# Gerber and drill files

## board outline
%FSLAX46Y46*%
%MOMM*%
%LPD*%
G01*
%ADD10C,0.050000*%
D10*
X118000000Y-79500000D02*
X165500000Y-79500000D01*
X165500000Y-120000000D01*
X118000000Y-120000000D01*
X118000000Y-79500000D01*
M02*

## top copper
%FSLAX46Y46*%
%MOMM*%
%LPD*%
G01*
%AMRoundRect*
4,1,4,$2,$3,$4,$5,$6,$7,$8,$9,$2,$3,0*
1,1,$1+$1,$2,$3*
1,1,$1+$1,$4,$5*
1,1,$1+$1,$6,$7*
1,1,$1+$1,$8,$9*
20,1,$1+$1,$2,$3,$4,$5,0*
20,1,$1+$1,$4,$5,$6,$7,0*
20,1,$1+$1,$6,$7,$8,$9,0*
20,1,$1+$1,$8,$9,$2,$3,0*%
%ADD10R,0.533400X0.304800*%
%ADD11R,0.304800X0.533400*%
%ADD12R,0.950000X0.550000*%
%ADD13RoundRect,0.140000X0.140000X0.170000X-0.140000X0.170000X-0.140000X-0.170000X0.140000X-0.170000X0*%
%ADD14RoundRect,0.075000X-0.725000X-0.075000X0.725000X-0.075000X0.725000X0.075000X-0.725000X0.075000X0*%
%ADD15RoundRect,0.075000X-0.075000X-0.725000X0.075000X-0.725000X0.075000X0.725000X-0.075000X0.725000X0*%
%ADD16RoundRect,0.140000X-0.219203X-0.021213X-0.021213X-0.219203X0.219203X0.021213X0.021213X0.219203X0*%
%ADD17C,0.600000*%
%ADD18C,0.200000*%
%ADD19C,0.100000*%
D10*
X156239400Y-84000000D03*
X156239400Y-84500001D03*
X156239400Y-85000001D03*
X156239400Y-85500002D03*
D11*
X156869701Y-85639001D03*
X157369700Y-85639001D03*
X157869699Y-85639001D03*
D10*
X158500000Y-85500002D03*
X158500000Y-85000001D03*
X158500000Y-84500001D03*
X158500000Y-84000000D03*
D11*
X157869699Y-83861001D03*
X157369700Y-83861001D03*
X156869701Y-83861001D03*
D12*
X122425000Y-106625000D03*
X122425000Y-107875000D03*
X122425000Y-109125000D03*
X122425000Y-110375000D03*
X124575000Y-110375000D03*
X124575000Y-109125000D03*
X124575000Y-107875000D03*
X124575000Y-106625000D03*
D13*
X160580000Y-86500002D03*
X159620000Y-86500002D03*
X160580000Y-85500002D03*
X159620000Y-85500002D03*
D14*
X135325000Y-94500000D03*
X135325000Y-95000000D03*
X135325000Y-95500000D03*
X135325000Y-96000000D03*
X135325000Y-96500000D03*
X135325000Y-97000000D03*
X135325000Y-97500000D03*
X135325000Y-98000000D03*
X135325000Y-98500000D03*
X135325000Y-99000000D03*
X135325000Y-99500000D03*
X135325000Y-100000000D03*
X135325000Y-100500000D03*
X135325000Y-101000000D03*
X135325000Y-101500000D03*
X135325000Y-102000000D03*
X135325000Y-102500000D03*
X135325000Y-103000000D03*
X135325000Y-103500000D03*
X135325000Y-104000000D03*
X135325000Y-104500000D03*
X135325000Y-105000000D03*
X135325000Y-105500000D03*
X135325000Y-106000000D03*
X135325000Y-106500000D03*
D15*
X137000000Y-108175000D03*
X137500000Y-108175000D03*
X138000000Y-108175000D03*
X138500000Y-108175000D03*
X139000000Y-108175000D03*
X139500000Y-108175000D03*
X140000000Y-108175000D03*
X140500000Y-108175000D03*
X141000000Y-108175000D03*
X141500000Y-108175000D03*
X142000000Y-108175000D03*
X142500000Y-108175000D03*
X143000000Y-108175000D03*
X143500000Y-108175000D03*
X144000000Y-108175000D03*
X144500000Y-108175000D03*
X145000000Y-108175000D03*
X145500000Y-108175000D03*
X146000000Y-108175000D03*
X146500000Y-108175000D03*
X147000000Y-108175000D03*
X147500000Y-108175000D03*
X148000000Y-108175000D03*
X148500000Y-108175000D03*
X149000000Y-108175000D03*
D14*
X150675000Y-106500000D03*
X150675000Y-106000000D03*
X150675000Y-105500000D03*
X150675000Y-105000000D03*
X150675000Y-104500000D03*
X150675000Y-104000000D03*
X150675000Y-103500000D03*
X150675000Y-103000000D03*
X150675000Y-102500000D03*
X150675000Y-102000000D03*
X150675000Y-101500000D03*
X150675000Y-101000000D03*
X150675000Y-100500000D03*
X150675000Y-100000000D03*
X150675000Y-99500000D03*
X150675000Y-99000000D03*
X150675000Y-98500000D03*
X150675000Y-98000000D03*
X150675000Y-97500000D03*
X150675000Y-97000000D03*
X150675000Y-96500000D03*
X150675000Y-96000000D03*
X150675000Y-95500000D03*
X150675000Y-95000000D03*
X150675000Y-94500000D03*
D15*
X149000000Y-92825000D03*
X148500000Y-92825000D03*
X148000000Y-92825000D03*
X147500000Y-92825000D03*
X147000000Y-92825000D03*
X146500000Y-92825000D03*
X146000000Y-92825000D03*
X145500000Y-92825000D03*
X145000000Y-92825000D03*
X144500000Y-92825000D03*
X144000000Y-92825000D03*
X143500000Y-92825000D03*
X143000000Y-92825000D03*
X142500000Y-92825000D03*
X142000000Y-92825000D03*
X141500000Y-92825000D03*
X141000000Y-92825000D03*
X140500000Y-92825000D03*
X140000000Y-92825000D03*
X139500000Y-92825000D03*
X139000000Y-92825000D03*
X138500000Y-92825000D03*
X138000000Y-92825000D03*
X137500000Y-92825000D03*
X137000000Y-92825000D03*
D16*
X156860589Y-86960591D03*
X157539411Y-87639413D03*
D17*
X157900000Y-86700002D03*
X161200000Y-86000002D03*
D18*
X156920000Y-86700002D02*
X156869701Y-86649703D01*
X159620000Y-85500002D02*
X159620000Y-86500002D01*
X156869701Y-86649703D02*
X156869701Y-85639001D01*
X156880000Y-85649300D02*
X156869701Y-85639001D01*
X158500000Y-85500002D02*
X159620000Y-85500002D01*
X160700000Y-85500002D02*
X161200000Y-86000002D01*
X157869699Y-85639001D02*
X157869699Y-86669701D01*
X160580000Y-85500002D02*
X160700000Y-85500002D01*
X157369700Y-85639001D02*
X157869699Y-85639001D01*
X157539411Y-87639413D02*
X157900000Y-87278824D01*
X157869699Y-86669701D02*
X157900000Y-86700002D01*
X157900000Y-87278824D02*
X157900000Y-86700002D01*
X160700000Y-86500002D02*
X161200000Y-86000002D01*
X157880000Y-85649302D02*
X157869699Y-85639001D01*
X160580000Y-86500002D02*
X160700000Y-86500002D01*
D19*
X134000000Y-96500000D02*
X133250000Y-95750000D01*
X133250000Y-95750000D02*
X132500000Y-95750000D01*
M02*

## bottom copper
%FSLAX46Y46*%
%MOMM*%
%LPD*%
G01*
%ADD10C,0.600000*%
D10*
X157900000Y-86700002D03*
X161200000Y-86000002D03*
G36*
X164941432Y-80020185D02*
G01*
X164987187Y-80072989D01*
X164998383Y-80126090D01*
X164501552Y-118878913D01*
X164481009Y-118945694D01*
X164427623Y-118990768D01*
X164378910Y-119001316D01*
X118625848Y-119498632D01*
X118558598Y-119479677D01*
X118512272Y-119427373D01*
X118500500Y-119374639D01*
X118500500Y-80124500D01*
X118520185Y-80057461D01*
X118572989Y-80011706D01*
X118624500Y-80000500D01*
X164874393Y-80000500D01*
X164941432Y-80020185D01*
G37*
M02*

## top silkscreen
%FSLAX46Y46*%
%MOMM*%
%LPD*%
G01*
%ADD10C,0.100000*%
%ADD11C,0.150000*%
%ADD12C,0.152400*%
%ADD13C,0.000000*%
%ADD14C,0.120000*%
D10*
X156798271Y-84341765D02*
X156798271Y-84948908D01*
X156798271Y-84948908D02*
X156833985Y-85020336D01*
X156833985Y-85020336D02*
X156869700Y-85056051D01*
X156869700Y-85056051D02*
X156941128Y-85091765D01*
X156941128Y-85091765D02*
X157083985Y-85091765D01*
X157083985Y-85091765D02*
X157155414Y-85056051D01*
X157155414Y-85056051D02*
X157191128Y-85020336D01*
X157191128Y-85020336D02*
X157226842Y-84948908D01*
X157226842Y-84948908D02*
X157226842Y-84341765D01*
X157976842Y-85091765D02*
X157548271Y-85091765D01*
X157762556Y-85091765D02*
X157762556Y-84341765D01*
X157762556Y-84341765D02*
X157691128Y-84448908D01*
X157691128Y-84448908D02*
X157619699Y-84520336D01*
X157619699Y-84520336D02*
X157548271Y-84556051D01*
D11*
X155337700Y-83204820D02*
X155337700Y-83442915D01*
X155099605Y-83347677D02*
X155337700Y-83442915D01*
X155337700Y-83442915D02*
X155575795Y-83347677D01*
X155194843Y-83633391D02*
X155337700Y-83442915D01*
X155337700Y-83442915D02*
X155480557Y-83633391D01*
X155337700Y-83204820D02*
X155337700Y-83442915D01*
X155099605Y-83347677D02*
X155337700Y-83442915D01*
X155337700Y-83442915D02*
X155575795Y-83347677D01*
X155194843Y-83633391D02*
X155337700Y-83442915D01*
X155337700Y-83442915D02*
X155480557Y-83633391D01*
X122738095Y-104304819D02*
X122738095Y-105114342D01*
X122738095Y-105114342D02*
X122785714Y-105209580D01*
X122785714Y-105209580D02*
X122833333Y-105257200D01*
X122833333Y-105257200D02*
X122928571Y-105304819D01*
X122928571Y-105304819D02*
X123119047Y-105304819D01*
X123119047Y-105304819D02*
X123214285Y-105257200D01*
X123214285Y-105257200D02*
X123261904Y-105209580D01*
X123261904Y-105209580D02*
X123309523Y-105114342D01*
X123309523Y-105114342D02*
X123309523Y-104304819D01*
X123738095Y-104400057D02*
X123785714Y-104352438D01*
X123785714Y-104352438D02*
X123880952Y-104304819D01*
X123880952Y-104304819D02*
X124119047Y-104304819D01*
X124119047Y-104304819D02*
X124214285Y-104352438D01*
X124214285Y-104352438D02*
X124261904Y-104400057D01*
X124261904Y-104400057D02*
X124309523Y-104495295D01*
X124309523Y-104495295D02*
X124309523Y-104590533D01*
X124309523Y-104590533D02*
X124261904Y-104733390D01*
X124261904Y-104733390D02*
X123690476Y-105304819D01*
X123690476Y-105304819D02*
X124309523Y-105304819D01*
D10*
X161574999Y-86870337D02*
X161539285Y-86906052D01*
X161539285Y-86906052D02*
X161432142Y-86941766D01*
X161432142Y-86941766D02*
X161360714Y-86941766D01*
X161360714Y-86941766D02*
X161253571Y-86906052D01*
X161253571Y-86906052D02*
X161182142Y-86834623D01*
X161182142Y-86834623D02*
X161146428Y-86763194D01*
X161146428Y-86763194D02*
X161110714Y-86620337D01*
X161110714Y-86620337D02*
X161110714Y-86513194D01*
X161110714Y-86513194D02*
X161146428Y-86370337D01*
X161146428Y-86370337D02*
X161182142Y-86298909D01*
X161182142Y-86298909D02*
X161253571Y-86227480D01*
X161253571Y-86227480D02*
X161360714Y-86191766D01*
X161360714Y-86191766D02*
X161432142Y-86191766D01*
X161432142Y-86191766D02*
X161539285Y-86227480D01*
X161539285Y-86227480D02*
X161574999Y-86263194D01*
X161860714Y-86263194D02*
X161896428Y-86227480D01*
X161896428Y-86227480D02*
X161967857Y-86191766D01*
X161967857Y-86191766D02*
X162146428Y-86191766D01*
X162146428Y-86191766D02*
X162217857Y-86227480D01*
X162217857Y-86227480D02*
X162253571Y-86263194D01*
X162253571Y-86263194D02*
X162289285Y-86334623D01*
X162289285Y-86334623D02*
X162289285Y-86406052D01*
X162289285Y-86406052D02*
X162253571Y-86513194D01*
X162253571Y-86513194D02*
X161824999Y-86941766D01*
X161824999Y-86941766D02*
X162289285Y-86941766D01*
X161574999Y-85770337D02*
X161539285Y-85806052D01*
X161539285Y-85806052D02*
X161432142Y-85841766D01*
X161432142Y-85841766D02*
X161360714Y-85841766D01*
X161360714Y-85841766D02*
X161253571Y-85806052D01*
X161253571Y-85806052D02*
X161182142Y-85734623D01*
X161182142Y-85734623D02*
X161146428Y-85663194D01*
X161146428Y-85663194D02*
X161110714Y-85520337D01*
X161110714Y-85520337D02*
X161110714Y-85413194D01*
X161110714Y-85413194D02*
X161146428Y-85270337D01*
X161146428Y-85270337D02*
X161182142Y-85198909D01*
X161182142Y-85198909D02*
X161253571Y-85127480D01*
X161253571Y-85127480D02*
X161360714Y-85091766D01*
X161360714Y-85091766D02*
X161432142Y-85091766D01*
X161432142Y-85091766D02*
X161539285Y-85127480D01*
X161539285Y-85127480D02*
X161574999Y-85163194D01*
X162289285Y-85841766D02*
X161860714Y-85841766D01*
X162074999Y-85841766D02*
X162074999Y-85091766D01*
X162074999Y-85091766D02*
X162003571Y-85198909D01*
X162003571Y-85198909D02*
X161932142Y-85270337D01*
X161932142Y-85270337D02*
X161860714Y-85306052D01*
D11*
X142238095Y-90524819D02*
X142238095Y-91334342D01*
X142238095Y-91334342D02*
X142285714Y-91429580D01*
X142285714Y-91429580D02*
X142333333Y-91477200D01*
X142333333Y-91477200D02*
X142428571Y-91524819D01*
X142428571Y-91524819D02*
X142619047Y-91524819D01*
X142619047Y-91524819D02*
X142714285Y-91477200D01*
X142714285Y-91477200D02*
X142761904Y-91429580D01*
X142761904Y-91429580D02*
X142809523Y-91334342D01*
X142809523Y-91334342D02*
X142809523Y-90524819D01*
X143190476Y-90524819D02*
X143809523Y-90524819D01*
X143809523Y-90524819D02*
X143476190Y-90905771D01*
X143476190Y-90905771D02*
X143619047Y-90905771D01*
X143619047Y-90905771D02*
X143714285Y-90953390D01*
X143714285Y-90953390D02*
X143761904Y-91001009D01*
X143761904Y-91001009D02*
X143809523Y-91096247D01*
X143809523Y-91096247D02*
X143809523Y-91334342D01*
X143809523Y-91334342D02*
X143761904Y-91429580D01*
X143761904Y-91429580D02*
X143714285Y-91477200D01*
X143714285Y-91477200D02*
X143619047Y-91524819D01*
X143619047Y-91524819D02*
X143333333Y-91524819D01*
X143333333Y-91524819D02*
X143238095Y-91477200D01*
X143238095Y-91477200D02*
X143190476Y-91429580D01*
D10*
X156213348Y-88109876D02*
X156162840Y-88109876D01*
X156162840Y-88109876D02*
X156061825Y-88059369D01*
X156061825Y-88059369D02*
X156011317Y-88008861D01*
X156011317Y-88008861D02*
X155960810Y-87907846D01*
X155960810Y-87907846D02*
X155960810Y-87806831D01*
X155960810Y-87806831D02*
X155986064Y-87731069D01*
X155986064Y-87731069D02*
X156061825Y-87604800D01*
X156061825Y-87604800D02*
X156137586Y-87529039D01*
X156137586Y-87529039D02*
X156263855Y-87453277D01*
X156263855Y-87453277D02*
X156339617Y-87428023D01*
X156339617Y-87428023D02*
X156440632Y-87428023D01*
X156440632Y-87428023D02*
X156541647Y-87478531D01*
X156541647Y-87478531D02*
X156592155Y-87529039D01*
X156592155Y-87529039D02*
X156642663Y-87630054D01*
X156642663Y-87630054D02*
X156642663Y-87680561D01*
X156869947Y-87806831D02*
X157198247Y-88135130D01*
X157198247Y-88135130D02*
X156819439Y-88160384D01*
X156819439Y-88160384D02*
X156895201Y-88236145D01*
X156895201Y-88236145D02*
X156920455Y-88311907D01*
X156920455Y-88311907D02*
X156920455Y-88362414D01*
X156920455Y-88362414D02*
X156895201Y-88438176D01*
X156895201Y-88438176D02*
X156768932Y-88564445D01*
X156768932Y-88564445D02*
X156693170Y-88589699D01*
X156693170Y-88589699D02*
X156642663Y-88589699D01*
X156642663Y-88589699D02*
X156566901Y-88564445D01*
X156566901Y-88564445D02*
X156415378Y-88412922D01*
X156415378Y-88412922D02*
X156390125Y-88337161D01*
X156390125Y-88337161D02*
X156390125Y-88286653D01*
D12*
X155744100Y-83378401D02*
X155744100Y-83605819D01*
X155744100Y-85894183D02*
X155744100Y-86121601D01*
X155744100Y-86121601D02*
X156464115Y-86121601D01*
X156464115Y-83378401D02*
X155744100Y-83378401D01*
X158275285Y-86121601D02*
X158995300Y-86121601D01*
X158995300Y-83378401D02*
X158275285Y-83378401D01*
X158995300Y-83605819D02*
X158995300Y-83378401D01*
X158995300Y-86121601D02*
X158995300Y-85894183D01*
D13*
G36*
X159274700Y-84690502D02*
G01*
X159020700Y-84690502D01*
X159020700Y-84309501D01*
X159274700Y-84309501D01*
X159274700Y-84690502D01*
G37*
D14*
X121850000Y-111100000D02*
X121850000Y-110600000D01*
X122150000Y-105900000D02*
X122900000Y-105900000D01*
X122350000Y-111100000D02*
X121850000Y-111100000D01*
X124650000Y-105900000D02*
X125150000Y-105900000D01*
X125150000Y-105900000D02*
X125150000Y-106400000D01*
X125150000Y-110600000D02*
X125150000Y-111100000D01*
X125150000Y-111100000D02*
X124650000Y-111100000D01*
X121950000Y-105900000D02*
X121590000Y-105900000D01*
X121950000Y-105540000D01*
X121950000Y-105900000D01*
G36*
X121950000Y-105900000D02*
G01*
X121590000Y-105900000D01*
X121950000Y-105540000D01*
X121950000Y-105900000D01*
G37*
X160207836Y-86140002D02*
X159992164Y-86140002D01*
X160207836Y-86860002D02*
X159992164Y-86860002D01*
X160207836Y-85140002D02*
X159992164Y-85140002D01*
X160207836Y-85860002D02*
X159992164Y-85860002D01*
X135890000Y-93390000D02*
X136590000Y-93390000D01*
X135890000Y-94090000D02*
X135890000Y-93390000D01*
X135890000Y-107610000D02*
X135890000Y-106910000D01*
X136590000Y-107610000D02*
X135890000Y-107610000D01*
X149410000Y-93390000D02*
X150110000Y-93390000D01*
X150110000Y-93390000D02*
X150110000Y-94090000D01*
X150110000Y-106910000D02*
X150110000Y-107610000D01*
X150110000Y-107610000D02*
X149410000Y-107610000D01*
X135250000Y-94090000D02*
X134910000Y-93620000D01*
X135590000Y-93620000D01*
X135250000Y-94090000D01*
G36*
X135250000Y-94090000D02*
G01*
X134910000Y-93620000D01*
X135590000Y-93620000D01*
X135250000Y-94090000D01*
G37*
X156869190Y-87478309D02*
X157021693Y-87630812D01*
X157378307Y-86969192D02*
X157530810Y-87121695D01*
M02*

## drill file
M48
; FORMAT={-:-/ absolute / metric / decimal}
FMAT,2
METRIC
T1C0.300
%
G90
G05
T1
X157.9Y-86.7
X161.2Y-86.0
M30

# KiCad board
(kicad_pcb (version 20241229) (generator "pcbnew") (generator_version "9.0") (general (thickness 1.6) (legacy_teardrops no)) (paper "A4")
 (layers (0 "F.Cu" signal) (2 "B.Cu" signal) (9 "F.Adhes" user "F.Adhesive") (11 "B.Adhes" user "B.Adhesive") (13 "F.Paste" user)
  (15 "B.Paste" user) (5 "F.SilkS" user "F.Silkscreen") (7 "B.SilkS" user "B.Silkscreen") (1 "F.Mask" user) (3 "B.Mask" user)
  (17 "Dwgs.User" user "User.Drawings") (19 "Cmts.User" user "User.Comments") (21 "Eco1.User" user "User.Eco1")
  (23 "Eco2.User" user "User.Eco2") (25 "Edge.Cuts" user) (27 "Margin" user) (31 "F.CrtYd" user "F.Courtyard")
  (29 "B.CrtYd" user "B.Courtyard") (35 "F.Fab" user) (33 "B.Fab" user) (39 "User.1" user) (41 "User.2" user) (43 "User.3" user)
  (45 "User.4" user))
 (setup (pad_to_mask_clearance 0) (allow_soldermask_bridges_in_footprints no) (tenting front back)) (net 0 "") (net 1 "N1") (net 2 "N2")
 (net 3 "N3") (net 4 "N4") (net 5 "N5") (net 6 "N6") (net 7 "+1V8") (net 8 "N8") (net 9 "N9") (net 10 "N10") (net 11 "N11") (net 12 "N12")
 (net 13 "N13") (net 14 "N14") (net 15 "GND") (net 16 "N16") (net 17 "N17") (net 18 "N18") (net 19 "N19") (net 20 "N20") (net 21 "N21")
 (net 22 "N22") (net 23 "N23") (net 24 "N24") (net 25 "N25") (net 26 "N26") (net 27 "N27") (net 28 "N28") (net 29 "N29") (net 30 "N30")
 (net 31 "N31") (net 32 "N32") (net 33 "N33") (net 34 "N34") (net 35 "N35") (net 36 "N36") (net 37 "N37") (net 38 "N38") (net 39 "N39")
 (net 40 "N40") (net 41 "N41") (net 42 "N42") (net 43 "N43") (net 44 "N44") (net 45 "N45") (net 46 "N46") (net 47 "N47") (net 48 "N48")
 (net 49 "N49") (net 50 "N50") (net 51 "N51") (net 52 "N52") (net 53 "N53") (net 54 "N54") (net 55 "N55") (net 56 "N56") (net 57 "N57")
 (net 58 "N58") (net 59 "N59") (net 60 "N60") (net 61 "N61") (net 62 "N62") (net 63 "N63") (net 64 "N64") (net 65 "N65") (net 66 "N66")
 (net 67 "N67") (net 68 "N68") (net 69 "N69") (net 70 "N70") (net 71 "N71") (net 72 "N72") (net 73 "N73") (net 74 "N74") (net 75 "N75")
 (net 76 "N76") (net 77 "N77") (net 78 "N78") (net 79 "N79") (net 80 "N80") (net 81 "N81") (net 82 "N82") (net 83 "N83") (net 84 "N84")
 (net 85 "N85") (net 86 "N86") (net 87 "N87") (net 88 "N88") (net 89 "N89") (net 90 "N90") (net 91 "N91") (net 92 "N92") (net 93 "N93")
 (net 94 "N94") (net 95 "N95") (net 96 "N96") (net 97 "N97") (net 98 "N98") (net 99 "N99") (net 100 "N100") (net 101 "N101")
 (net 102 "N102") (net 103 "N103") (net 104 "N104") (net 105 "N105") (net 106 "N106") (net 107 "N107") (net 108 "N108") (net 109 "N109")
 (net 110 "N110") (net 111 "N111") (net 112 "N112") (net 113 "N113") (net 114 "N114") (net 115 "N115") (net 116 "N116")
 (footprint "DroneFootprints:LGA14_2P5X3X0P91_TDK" (layer "F.Cu") (at 157.3697 84.750001)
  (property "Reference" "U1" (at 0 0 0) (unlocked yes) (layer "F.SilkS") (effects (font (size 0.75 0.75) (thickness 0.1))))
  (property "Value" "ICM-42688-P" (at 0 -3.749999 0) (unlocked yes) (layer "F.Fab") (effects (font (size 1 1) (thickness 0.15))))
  (fp_line (start -1.6256 -1.3716) (end -1.6256 -1.144182) (stroke (width 0.1524) (type solid)) (layer "F.SilkS"))
  (fp_line (start -1.6256 1.144182) (end -1.6256 1.3716) (stroke (width 0.1524) (type solid)) (layer "F.SilkS"))
  (fp_line (start -1.6256 1.3716) (end -0.905585 1.3716) (stroke (width 0.1524) (type solid)) (layer "F.SilkS"))
  (fp_line (start -0.905585 -1.3716) (end -1.6256 -1.3716) (stroke (width 0.1524) (type solid)) (layer "F.SilkS"))
  (fp_line (start 0.905585 1.3716) (end 1.6256 1.3716) (stroke (width 0.1524) (type solid)) (layer "F.SilkS"))
  (fp_line (start 1.6256 -1.3716) (end 0.905585 -1.3716) (stroke (width 0.1524) (type solid)) (layer "F.SilkS"))
  (fp_line (start 1.6256 -1.144182) (end 1.6256 -1.3716) (stroke (width 0.1524) (type solid)) (layer "F.SilkS"))
  (fp_line (start 1.6256 1.3716) (end 1.6256 1.144182) (stroke (width 0.1524) (type solid)) (layer "F.SilkS"))
  (fp_poly
   (pts (xy 1.905 -0.4405) (xy 1.905 -0.059499) (xy 1.651 -0.059499) (xy 1.651 -0.4405)) (stroke (width 0) (type solid)) (fill yes)
   (layer "F.SilkS"))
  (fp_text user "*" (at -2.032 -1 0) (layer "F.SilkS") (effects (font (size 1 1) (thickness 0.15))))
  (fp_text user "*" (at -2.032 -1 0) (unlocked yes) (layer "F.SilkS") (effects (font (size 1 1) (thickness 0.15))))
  (pad "1" smd rect (at -1.1303 -0.750001 90) (size 0.3048 0.5334) (layers "F.Cu" "F.Mask" "F.Paste") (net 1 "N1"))
  (pad "2" smd rect (at -1.1303 -0.25 90) (size 0.3048 0.5334) (layers "F.Cu" "F.Mask" "F.Paste") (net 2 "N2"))
  (pad "3" smd rect (at -1.1303 0.25 90) (size 0.3048 0.5334) (layers "F.Cu" "F.Mask" "F.Paste") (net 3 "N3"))
  (pad "4" smd rect (at -1.1303 0.750001 90) (size 0.3048 0.5334) (layers "F.Cu" "F.Mask" "F.Paste") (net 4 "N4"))
  (pad "5" smd rect (at -0.499999 0.889) (size 0.3048 0.5334) (layers "F.Cu" "F.Mask" "F.Paste") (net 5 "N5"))
  (pad "6" smd rect (at 0 0.889) (size 0.3048 0.5334) (layers "F.Cu" "F.Mask" "F.Paste") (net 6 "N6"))
  (pad "7" smd rect (at 0.499999 0.889) (size 0.3048 0.5334) (layers "F.Cu" "F.Mask" "F.Paste") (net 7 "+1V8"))
  (pad "8" smd rect (at 1.1303 0.750001 90) (size 0.3048 0.5334) (layers "F.Cu" "F.Mask" "F.Paste") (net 7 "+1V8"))
  (pad "9" smd rect (at 1.1303 0.25 90) (size 0.3048 0.5334) (layers "F.Cu" "F.Mask" "F.Paste") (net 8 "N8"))
  (pad "10" smd rect (at 1.1303 -0.25 90) (size 0.3048 0.5334) (layers "F.Cu" "F.Mask" "F.Paste") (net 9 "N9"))
  (pad "11" smd rect (at 1.1303 -0.750001 90) (size 0.3048 0.5334) (layers "F.Cu" "F.Mask" "F.Paste") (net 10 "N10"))
  (pad "12" smd rect (at 0.499999 -0.889) (size 0.3048 0.5334) (layers "F.Cu" "F.Mask" "F.Paste") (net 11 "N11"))
  (pad "13" smd rect (at 0 -0.889) (size 0.3048 0.5334) (layers "F.Cu" "F.Mask" "F.Paste") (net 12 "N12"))
  (pad "14" smd rect (at -0.499999 -0.889) (size 0.3048 0.5334) (layers "F.Cu" "F.Mask" "F.Paste") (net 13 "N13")))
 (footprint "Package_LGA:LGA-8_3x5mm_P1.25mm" (layer "F.Cu") (at 123.5 108.5)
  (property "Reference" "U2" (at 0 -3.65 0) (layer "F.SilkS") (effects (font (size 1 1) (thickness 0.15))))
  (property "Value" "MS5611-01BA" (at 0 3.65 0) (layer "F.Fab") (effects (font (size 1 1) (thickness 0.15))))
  (fp_line (start -1.65 2.6) (end -1.65 2.1) (stroke (width 0.12) (type solid)) (layer "F.SilkS"))
  (fp_line (start -1.35 -2.6) (end -0.6 -2.6) (stroke (width 0.12) (type solid)) (layer "F.SilkS"))
  (fp_line (start -1.15 2.6) (end -1.65 2.6) (stroke (width 0.12) (type solid)) (layer "F.SilkS"))
  (fp_line (start 1.15 -2.6) (end 1.65 -2.6) (stroke (width 0.12) (type solid)) (layer "F.SilkS"))
  (fp_line (start 1.65 -2.6) (end 1.65 -2.1) (stroke (width 0.12) (type solid)) (layer "F.SilkS"))
  (fp_line (start 1.65 2.1) (end 1.65 2.6) (stroke (width 0.12) (type solid)) (layer "F.SilkS"))
  (fp_line (start 1.65 2.6) (end 1.15 2.6) (stroke (width 0.12) (type solid)) (layer "F.SilkS"))
  (fp_poly
   (pts (xy -1.55 -2.6) (xy -1.91 -2.6) (xy -1.55 -2.96) (xy -1.55 -2.6)) (stroke (width 0.12) (type solid)) (fill yes) (layer "F.SilkS"))
  (pad "1" smd rect (at -1.075 -1.875) (size 0.95 0.55) (layers "F.Cu" "F.Mask" "F.Paste") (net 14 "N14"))
  (pad "2" smd rect (at -1.075 -0.625) (size 0.95 0.55) (layers "F.Cu" "F.Mask" "F.Paste") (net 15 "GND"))
  (pad "3" smd rect (at -1.075 0.625) (size 0.95 0.55) (layers "F.Cu" "F.Mask" "F.Paste") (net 15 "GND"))
  (pad "4" smd rect (at -1.075 1.875) (size 0.95 0.55) (layers "F.Cu" "F.Mask" "F.Paste") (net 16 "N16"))
  (pad "5" smd rect (at 1.075 1.875) (size 0.95 0.55) (layers "F.Cu" "F.Mask" "F.Paste") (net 16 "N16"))
  (pad "6" smd rect (at 1.075 0.625) (size 0.95 0.55) (layers "F.Cu" "F.Mask" "F.Paste") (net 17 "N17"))
  (pad "7" smd rect (at 1.075 -0.625) (size 0.95 0.55) (layers "F.Cu" "F.Mask" "F.Paste") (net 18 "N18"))
  (pad "8" smd rect (at 1.075 -1.875) (size 0.95 0.55) (layers "F.Cu" "F.Mask" "F.Paste") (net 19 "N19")))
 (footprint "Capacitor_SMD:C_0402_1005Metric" (layer "F.Cu") (at 160.1 86.500002 180)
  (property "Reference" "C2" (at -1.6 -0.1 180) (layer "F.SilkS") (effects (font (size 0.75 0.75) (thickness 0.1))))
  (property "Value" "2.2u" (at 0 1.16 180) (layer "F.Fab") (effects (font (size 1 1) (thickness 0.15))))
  (fp_line (start -0.107836 0.36) (end 0.107836 0.36) (stroke (width 0.12) (type solid)) (layer "F.SilkS"))
  (fp_line (start -0.107836 -0.36) (end 0.107836 -0.36) (stroke (width 0.12) (type solid)) (layer "F.SilkS"))
  (pad "1" smd roundrect (at -0.48 0 180) (size 0.56 0.62) (layers "F.Cu" "F.Mask" "F.Paste") (roundrect_rratio 0.25) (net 15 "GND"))
  (pad "2" smd roundrect (at 0.48 0 180) (size 0.56 0.62) (layers "F.Cu" "F.Mask" "F.Paste") (roundrect_rratio 0.25) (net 7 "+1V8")))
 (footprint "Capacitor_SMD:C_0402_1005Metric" (layer "F.Cu") (at 160.1 85.500002 180)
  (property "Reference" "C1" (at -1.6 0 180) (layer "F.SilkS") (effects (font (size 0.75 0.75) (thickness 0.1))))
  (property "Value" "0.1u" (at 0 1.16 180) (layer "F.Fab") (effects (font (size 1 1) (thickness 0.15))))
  (fp_line (start -0.107836 0.36) (end 0.107836 0.36) (stroke (width 0.12) (type solid)) (layer "F.SilkS"))
  (fp_line (start -0.107836 -0.36) (end 0.107836 -0.36) (stroke (width 0.12) (type solid)) (layer "F.SilkS"))
  (pad "1" smd roundrect (at -0.48 0 180) (size 0.56 0.62) (layers "F.Cu" "F.Mask" "F.Paste") (roundrect_rratio 0.25) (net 15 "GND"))
  (pad "2" smd roundrect (at 0.48 0 180) (size 0.56 0.62) (layers "F.Cu" "F.Mask" "F.Paste") (roundrect_rratio 0.25) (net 7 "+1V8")))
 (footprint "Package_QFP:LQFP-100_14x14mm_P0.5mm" (layer "F.Cu") (at 143 100.5)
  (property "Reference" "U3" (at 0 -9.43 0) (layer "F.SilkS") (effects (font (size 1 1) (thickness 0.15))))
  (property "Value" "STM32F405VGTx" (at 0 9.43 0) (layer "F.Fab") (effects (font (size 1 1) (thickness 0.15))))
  (fp_line (start -7.11 -7.11) (end -6.41 -7.11) (stroke (width 0.12) (type solid)) (layer "F.SilkS"))
  (fp_line (start -7.11 -6.41) (end -7.11 -7.11) (stroke (width 0.12) (type solid)) (layer "F.SilkS"))
  (fp_line (start -7.11 7.11) (end -7.11 6.41) (stroke (width 0.12) (type solid)) (layer "F.SilkS"))
  (fp_line (start -6.41 7.11) (end -7.11 7.11) (stroke (width 0.12) (type solid)) (layer "F.SilkS"))
  (fp_line (start 6.41 -7.11) (end 7.11 -7.11) (stroke (width 0.12) (type solid)) (layer "F.SilkS"))
  (fp_line (start 7.11 -7.11) (end 7.11 -6.41) (stroke (width 0.12) (type solid)) (layer "F.SilkS"))
  (fp_line (start 7.11 6.41) (end 7.11 7.11) (stroke (width 0.12) (type solid)) (layer "F.SilkS"))
  (fp_line (start 7.11 7.11) (end 6.41 7.11) (stroke (width 0.12) (type solid)) (layer "F.SilkS"))
  (fp_poly (pts (xy -7.75 -6.41) (xy -8.09 -6.88) (xy -7.41 -6.88)) (stroke (width 0.12) (type solid)) (fill yes) (layer "F.SilkS"))
  (pad "1" smd roundrect (at -7.675 -6) (size 1.6 0.3) (layers "F.Cu" "F.Mask" "F.Paste") (roundrect_rratio 0.25) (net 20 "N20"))
  (pad "2" smd roundrect (at -7.675 -5.5) (size 1.6 0.3) (layers "F.Cu" "F.Mask" "F.Paste") (roundrect_rratio 0.25) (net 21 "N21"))
  (pad "3" smd roundrect (at -7.675 -5) (size 1.6 0.3) (layers "F.Cu" "F.Mask" "F.Paste") (roundrect_rratio 0.25) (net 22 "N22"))
  (pad "4" smd roundrect (at -7.675 -4.5) (size 1.6 0.3) (layers "F.Cu" "F.Mask" "F.Paste") (roundrect_rratio 0.25) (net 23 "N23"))
  (pad "5" smd roundrect (at -7.675 -4) (size 1.6 0.3) (layers "F.Cu" "F.Mask" "F.Paste") (roundrect_rratio 0.25) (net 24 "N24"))
  (pad "6" smd roundrect (at -7.675 -3.5) (size 1.6 0.3) (layers "F.Cu" "F.Mask" "F.Paste") (roundrect_rratio 0.25) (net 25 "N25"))
  (pad "7" smd roundrect (at -7.675 -3) (size 1.6 0.3) (layers "F.Cu" "F.Mask" "F.Paste") (roundrect_rratio 0.25) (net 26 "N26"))
  (pad "8" smd roundrect (at -7.675 -2.5) (size 1.6 0.3) (layers "F.Cu" "F.Mask" "F.Paste") (roundrect_rratio 0.25) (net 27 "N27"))
  (pad "9" smd roundrect (at -7.675 -2) (size 1.6 0.3) (layers "F.Cu" "F.Mask" "F.Paste") (roundrect_rratio 0.25) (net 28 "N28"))
  (pad "10" smd roundrect (at -7.675 -1.5) (size 1.6 0.3) (layers "F.Cu" "F.Mask" "F.Paste") (roundrect_rratio 0.25) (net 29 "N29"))
  (pad "11" smd roundrect (at -7.675 -1) (size 1.6 0.3) (layers "F.Cu" "F.Mask" "F.Paste") (roundrect_rratio 0.25) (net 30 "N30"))
  (pad "12" smd roundrect (at -7.675 -0.5) (size 1.6 0.3) (layers "F.Cu" "F.Mask" "F.Paste") (roundrect_rratio 0.25) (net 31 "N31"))
  (pad "13" smd roundrect (at -7.675 0) (size 1.6 0.3) (layers "F.Cu" "F.Mask" "F.Paste") (roundrect_rratio 0.25) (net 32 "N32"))
  (pad "14" smd roundrect (at -7.675 0.5) (size 1.6 0.3) (layers "F.Cu" "F.Mask" "F.Paste") (roundrect_rratio 0.25) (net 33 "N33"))
  (pad "15" smd roundrect (at -7.675 1) (size 1.6 0.3) (layers "F.Cu" "F.Mask" "F.Paste") (roundrect_rratio 0.25) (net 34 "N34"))
  (pad "16" smd roundrect (at -7.675 1.5) (size 1.6 0.3) (layers "F.Cu" "F.Mask" "F.Paste") (roundrect_rratio 0.25) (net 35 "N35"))
  (pad "17" smd roundrect (at -7.675 2) (size 1.6 0.3) (layers "F.Cu" "F.Mask" "F.Paste") (roundrect_rratio 0.25) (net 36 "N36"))
  (pad "18" smd roundrect (at -7.675 2.5) (size 1.6 0.3) (layers "F.Cu" "F.Mask" "F.Paste") (roundrect_rratio 0.25) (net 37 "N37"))
  (pad "19" smd roundrect (at -7.675 3) (size 1.6 0.3) (layers "F.Cu" "F.Mask" "F.Paste") (roundrect_rratio 0.25) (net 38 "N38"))
  (pad "20" smd roundrect (at -7.675 3.5) (size 1.6 0.3) (layers "F.Cu" "F.Mask" "F.Paste") (roundrect_rratio 0.25) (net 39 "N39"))
  (pad "21" smd roundrect (at -7.675 4) (size 1.6 0.3) (layers "F.Cu" "F.Mask" "F.Paste") (roundrect_rratio 0.25) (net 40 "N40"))
  (pad "22" smd roundrect (at -7.675 4.5) (size 1.6 0.3) (layers "F.Cu" "F.Mask" "F.Paste") (roundrect_rratio 0.25) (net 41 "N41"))
  (pad "23" smd roundrect (at -7.675 5) (size 1.6 0.3) (layers "F.Cu" "F.Mask" "F.Paste") (roundrect_rratio 0.25) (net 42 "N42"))
  (pad "24" smd roundrect (at -7.675 5.5) (size 1.6 0.3) (layers "F.Cu" "F.Mask" "F.Paste") (roundrect_rratio 0.25) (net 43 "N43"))
  (pad "25" smd roundrect (at -7.675 6) (size 1.6 0.3) (layers "F.Cu" "F.Mask" "F.Paste") (roundrect_rratio 0.25) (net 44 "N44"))
  (pad "26" smd roundrect (at -6 7.675) (size 0.3 1.6) (layers "F.Cu" "F.Mask" "F.Paste") (roundrect_rratio 0.25) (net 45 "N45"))
  (pad "27" smd roundrect (at -5.5 7.675) (size 0.3 1.6) (layers "F.Cu" "F.Mask" "F.Paste") (roundrect_rratio 0.25) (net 29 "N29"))
  (pad "28" smd roundrect (at -5 7.675) (size 0.3 1.6) (layers "F.Cu" "F.Mask" "F.Paste") (roundrect_rratio 0.25) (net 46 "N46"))
  (pad "29" smd roundrect (at -4.5 7.675) (size 0.3 1.6) (layers "F.Cu" "F.Mask" "F.Paste") (roundrect_rratio 0.25) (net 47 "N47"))
  (pad "30" smd roundrect (at -4 7.675) (size 0.3 1.6) (layers "F.Cu" "F.Mask" "F.Paste") (roundrect_rratio 0.25) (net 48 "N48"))
  (pad "31" smd roundrect (at -3.5 7.675) (size 0.3 1.6) (layers "F.Cu" "F.Mask" "F.Paste") (roundrect_rratio 0.25) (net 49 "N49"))
  (pad "32" smd roundrect (at -3 7.675) (size 0.3 1.6) (layers "F.Cu" "F.Mask" "F.Paste") (roundrect_rratio 0.25) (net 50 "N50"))
  (pad "33" smd roundrect (at -2.5 7.675) (size 0.3 1.6) (layers "F.Cu" "F.Mask" "F.Paste") (roundrect_rratio 0.25) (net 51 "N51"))
  (pad "34" smd roundrect (at -2 7.675) (size 0.3 1.6) (layers "F.Cu" "F.Mask" "F.Paste") (roundrect_rratio 0.25) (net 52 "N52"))
  (pad "35" smd roundrect (at -1.5 7.675) (size 0.3 1.6) (layers "F.Cu" "F.Mask" "F.Paste") (roundrect_rratio 0.25) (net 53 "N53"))
  (pad "36" smd roundrect (at -1 7.675) (size 0.3 1.6) (layers "F.Cu" "F.Mask" "F.Paste") (roundrect_rratio 0.25) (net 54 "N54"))
  (pad "37" smd roundrect (at -0.5 7.675) (size 0.3 1.6) (layers "F.Cu" "F.Mask" "F.Paste") (roundrect_rratio 0.25) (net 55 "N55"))
  (pad "38" smd roundrect (at 0 7.675) (size 0.3 1.6) (layers "F.Cu" "F.Mask" "F.Paste") (roundrect_rratio 0.25) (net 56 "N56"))
  (pad "39" smd roundrect (at 0.5 7.675) (size 0.3 1.6) (layers "F.Cu" "F.Mask" "F.Paste") (roundrect_rratio 0.25) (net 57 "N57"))
  (pad "40" smd roundrect (at 1 7.675) (size 0.3 1.6) (layers "F.Cu" "F.Mask" "F.Paste") (roundrect_rratio 0.25) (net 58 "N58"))
  (pad "41" smd roundrect (at 1.5 7.675) (size 0.3 1.6) (layers "F.Cu" "F.Mask" "F.Paste") (roundrect_rratio 0.25) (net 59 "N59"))
  (pad "42" smd roundrect (at 2 7.675) (size 0.3 1.6) (layers "F.Cu" "F.Mask" "F.Paste") (roundrect_rratio 0.25) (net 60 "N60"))
  (pad "43" smd roundrect (at 2.5 7.675) (size 0.3 1.6) (layers "F.Cu" "F.Mask" "F.Paste") (roundrect_rratio 0.25) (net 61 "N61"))
  (pad "44" smd roundrect (at 3 7.675) (size 0.3 1.6) (layers "F.Cu" "F.Mask" "F.Paste") (roundrect_rratio 0.25) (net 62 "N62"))
  (pad "45" smd roundrect (at 3.5 7.675) (size 0.3 1.6) (layers "F.Cu" "F.Mask" "F.Paste") (roundrect_rratio 0.25) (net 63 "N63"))
  (pad "46" smd roundrect (at 4 7.675) (size 0.3 1.6) (layers "F.Cu" "F.Mask" "F.Paste") (roundrect_rratio 0.25) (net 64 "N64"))
  (pad "47" smd roundrect (at 4.5 7.675) (size 0.3 1.6) (layers "F.Cu" "F.Mask" "F.Paste") (roundrect_rratio 0.25) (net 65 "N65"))
  (pad "48" smd roundrect (at 5 7.675) (size 0.3 1.6) (layers "F.Cu" "F.Mask" "F.Paste") (roundrect_rratio 0.25) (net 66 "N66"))
  (pad "49" smd roundrect (at 5.5 7.675) (size 0.3 1.6) (layers "F.Cu" "F.Mask" "F.Paste") (roundrect_rratio 0.25) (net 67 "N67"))
  (pad "50" smd roundrect (at 6 7.675) (size 0.3 1.6) (layers "F.Cu" "F.Mask" "F.Paste") (roundrect_rratio 0.25) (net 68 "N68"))
  (pad "51" smd roundrect (at 7.675 6) (size 1.6 0.3) (layers "F.Cu" "F.Mask" "F.Paste") (roundrect_rratio 0.25) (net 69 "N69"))
  (pad "52" smd roundrect (at 7.675 5.5) (size 1.6 0.3) (layers "F.Cu" "F.Mask" "F.Paste") (roundrect_rratio 0.25) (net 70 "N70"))
  (pad "53" smd roundrect (at 7.675 5) (size 1.6 0.3) (layers "F.Cu" "F.Mask" "F.Paste") (roundrect_rratio 0.25) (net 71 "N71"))
  (pad "54" smd roundrect (at 7.675 4.5) (size 1.6 0.3) (layers "F.Cu" "F.Mask" "F.Paste") (roundrect_rratio 0.25) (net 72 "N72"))
  (pad "55" smd roundrect (at 7.675 4) (size 1.6 0.3) (layers "F.Cu" "F.Mask" "F.Paste") (roundrect_rratio 0.25) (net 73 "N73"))
  (pad "56" smd roundrect (at 7.675 3.5) (size 1.6 0.3) (layers "F.Cu" "F.Mask" "F.Paste") (roundrect_rratio 0.25) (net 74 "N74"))
  (pad "57" smd roundrect (at 7.675 3) (size 1.6 0.3) (layers "F.Cu" "F.Mask" "F.Paste") (roundrect_rratio 0.25) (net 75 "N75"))
  (pad "58" smd roundrect (at 7.675 2.5) (size 1.6 0.3) (layers "F.Cu" "F.Mask" "F.Paste") (roundrect_rratio 0.25) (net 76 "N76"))
  (pad "59" smd roundrect (at 7.675 2) (size 1.6 0.3) (layers "F.Cu" "F.Mask" "F.Paste") (roundrect_rratio 0.25) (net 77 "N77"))
  (pad "60" smd roundrect (at 7.675 1.5) (size 1.6 0.3) (layers "F.Cu" "F.Mask" "F.Paste") (roundrect_rratio 0.25) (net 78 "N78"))
  (pad "61" smd roundrect (at 7.675 1) (size 1.6 0.3) (layers "F.Cu" "F.Mask" "F.Paste") (roundrect_rratio 0.25) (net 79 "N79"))
  (pad "62" smd roundrect (at 7.675 0.5) (size 1.6 0.3) (layers "F.Cu" "F.Mask" "F.Paste") (roundrect_rratio 0.25) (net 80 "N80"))
  (pad "63" smd roundrect (at 7.675 0) (size 1.6 0.3) (layers "F.Cu" "F.Mask" "F.Paste") (roundrect_rratio 0.25) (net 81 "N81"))
  (pad "64" smd roundrect (at 7.675 -0.5) (size 1.6 0.3) (layers "F.Cu" "F.Mask" "F.Paste") (roundrect_rratio 0.25) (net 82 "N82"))
  (pad "65" smd roundrect (at 7.675 -1) (size 1.6 0.3) (layers "F.Cu" "F.Mask" "F.Paste") (roundrect_rratio 0.25) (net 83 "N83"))
  (pad "66" smd roundrect (at 7.675 -1.5) (size 1.6 0.3) (layers "F.Cu" "F.Mask" "F.Paste") (roundrect_rratio 0.25) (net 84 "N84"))
  (pad "67" smd roundrect (at 7.675 -2) (size 1.6 0.3) (layers "F.Cu" "F.Mask" "F.Paste") (roundrect_rratio 0.25) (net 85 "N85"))
  (pad "68" smd roundrect (at 7.675 -2.5) (size 1.6 0.3) (layers "F.Cu" "F.Mask" "F.Paste") (roundrect_rratio 0.25) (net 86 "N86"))
  (pad "69" smd roundrect (at 7.675 -3) (size 1.6 0.3) (layers "F.Cu" "F.Mask" "F.Paste") (roundrect_rratio 0.25) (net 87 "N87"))
  (pad "70" smd roundrect (at 7.675 -3.5) (size 1.6 0.3) (layers "F.Cu" "F.Mask" "F.Paste") (roundrect_rratio 0.25) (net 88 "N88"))
  (pad "71" smd roundrect (at 7.675 -4) (size 1.6 0.3) (layers "F.Cu" "F.Mask" "F.Paste") (roundrect_rratio 0.25) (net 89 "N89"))
  (pad "72" smd roundrect (at 7.675 -4.5) (size 1.6 0.3) (layers "F.Cu" "F.Mask" "F.Paste") (roundrect_rratio 0.25) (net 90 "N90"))
  (pad "73" smd roundrect (at 7.675 -5) (size 1.6 0.3) (layers "F.Cu" "F.Mask" "F.Paste") (roundrect_rratio 0.25) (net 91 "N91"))
  (pad "74" smd roundrect (at 7.675 -5.5) (size 1.6 0.3) (layers "F.Cu" "F.Mask" "F.Paste") (roundrect_rratio 0.25) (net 29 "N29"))
  (pad "75" smd roundrect (at 7.675 -6) (size 1.6 0.3) (layers "F.Cu" "F.Mask" "F.Paste") (roundrect_rratio 0.25) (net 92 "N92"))
  (pad "76" smd roundrect (at 6 -7.675) (size 0.3 1.6) (layers "F.Cu" "F.Mask" "F.Paste") (roundrect_rratio 0.25) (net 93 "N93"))
  (pad "77" smd roundrect (at 5.5 -7.675) (size 0.3 1.6) (layers "F.Cu" "F.Mask" "F.Paste") (roundrect_rratio 0.25) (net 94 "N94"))
  (pad "78" smd roundrect (at 5 -7.675) (size 0.3 1.6) (layers "F.Cu" "F.Mask" "F.Paste") (roundrect_rratio 0.25) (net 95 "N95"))
  (pad "79" smd roundrect (at 4.5 -7.675) (size 0.3 1.6) (layers "F.Cu" "F.Mask" "F.Paste") (roundrect_rratio 0.25) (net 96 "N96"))
  (pad "80" smd roundrect (at 4 -7.675) (size 0.3 1.6) (layers "F.Cu" "F.Mask" "F.Paste") (roundrect_rratio 0.25) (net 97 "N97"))
  (pad "81" smd roundrect (at 3.5 -7.675) (size 0.3 1.6) (layers "F.Cu" "F.Mask" "F.Paste") (roundrect_rratio 0.25) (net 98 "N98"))
  (pad "82" smd roundrect (at 3 -7.675) (size 0.3 1.6) (layers "F.Cu" "F.Mask" "F.Paste") (roundrect_rratio 0.25) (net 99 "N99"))
  (pad "83" smd roundrect (at 2.5 -7.675) (size 0.3 1.6) (layers "F.Cu" "F.Mask" "F.Paste") (roundrect_rratio 0.25) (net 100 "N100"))
  (pad "84" smd roundrect (at 2 -7.675) (size 0.3 1.6) (layers "F.Cu" "F.Mask" "F.Paste") (roundrect_rratio 0.25) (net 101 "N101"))
  (pad "85" smd roundrect (at 1.5 -7.675) (size 0.3 1.6) (layers "F.Cu" "F.Mask" "F.Paste") (roundrect_rratio 0.25) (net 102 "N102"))
  (pad "86" smd roundrect (at 1 -7.675) (size 0.3 1.6) (layers "F.Cu" "F.Mask" "F.Paste") (roundrect_rratio 0.25) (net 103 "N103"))
  (pad "87" smd roundrect (at 0.5 -7.675) (size 0.3 1.6) (layers "F.Cu" "F.Mask" "F.Paste") (roundrect_rratio 0.25) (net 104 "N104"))
  (pad "88" smd roundrect (at 0 -7.675) (size 0.3 1.6) (layers "F.Cu" "F.Mask" "F.Paste") (roundrect_rratio 0.25) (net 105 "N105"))
  (pad "89" smd roundrect (at -0.5 -7.675) (size 0.3 1.6) (layers "F.Cu" "F.Mask" "F.Paste") (roundrect_rratio 0.25) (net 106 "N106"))
  (pad "90" smd roundrect (at -1 -7.675) (size 0.3 1.6) (layers "F.Cu" "F.Mask" "F.Paste") (roundrect_rratio 0.25) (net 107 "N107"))
  (pad "91" smd roundrect (at -1.5 -7.675) (size 0.3 1.6) (layers "F.Cu" "F.Mask" "F.Paste") (roundrect_rratio 0.25) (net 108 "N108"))
  (pad "92" smd roundrect (at -2 -7.675) (size 0.3 1.6) (layers "F.Cu" "F.Mask" "F.Paste") (roundrect_rratio 0.25) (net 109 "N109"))
  (pad "93" smd roundrect (at -2.5 -7.675) (size 0.3 1.6) (layers "F.Cu" "F.Mask" "F.Paste") (roundrect_rratio 0.25) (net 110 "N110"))
  (pad "94" smd roundrect (at -3 -7.675) (size 0.3 1.6) (layers "F.Cu" "F.Mask" "F.Paste") (roundrect_rratio 0.25) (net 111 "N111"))
  (pad "95" smd roundrect (at -3.5 -7.675) (size 0.3 1.6) (layers "F.Cu" "F.Mask" "F.Paste") (roundrect_rratio 0.25) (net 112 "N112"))
  (pad "96" smd roundrect (at -4 -7.675) (size 0.3 1.6) (layers "F.Cu" "F.Mask" "F.Paste") (roundrect_rratio 0.25) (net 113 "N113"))
  (pad "97" smd roundrect (at -4.5 -7.675) (size 0.3 1.6) (layers "F.Cu" "F.Mask" "F.Paste") (roundrect_rratio 0.25) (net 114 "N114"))
  (pad "98" smd roundrect (at -5 -7.675) (size 0.3 1.6) (layers "F.Cu" "F.Mask" "F.Paste") (roundrect_rratio 0.25) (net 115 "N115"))
  (pad "99" smd roundrect (at -5.5 -7.675) (size 0.3 1.6) (layers "F.Cu" "F.Mask" "F.Paste") (roundrect_rratio 0.25) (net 29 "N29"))
  (pad "100" smd roundrect (at -6 -7.675) (size 0.3 1.6) (layers "F.Cu" "F.Mask" "F.Paste") (roundrect_rratio 0.25) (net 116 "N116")))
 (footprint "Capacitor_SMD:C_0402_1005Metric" (layer "F.Cu") (at 157.2 87.300002 -45)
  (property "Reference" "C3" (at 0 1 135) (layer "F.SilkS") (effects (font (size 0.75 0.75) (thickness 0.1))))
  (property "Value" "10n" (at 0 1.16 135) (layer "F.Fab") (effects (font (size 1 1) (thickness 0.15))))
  (fp_line (start -0.107836 0.36) (end 0.107836 0.36) (stroke (width 0.12) (type solid)) (layer "F.SilkS"))
  (fp_line (start -0.107836 -0.36) (end 0.107836 -0.36) (stroke (width 0.12) (type solid)) (layer "F.SilkS"))
  (pad "1" smd roundrect (at -0.48 0 315) (size 0.56 0.62) (layers "F.Cu" "F.Mask" "F.Paste") (roundrect_rratio 0.25) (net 7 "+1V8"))
  (pad "2" smd roundrect (at 0.48 0 315) (size 0.56 0.62) (layers "F.Cu" "F.Mask" "F.Paste") (roundrect_rratio 0.25) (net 15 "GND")))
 (gr_rect (start 118 79.5) (end 165.5 120) (stroke (width 0.05) (type default)) (fill no) (layer "Edge.Cuts"))
 (segment (start 156.92 86.700002) (end 156.869701 86.649703) (width 0.2) (layer "F.Cu") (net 7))
 (segment (start 159.62 85.500002) (end 159.62 86.500002) (width 0.2) (layer "F.Cu") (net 7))
 (segment (start 156.869701 86.649703) (end 156.869701 85.639001) (width 0.2) (layer "F.Cu") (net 7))
 (segment (start 156.88 85.6493) (end 156.869701 85.639001) (width 0.2) (layer "F.Cu") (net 7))
 (segment (start 158.5 85.500002) (end 159.62 85.500002) (width 0.2) (layer "F.Cu") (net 7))
 (segment (start 160.7 85.500002) (end 161.2 86.000002) (width 0.2) (layer "F.Cu") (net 15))
 (segment (start 157.869699 85.639001) (end 157.869699 86.669701) (width 0.2) (layer "F.Cu") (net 15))
 (segment (start 160.58 85.500002) (end 160.7 85.500002) (width 0.2) (layer "F.Cu") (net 15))
 (segment (start 157.3697 85.639001) (end 157.869699 85.639001) (width 0.2) (layer "F.Cu") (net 15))
 (segment (start 157.539411 87.639413) (end 157.9 87.278824) (width 0.2) (layer "F.Cu") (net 15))
 (segment (start 157.869699 86.669701) (end 157.9 86.700002) (width 0.2) (layer "F.Cu") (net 15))
 (segment (start 157.9 87.278824) (end 157.9 86.700002) (width 0.2) (layer "F.Cu") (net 15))
 (segment (start 160.7 86.500002) (end 161.2 86.000002) (width 0.2) (layer "F.Cu") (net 15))
 (segment (start 157.88 85.649302) (end 157.869699 85.639001) (width 0.2) (layer "F.Cu") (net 15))
 (segment (start 160.58 86.500002) (end 160.7 86.500002) (width 0.2) (layer "F.Cu") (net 15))
 (via (at 157.9 86.700002) (size 0.6) (drill 0.3) (layers "F.Cu" "B.Cu") (free yes) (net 15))
 (via (at 161.2 86.000002) (size 0.6) (drill 0.3) (layers "F.Cu" "B.Cu") (free yes) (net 15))
 (segment (start 134 96.5) (end 133.25 95.75) (width 0.1) (layer "F.Cu") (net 18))
 (segment (start 133.25 95.75) (end 132.5 95.75) (width 0.1) (layer "F.Cu") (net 18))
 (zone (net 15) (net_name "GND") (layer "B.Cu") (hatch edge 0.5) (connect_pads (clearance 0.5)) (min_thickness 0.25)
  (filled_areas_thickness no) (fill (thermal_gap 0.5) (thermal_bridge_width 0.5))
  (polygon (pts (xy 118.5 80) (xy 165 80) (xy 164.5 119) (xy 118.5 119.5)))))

